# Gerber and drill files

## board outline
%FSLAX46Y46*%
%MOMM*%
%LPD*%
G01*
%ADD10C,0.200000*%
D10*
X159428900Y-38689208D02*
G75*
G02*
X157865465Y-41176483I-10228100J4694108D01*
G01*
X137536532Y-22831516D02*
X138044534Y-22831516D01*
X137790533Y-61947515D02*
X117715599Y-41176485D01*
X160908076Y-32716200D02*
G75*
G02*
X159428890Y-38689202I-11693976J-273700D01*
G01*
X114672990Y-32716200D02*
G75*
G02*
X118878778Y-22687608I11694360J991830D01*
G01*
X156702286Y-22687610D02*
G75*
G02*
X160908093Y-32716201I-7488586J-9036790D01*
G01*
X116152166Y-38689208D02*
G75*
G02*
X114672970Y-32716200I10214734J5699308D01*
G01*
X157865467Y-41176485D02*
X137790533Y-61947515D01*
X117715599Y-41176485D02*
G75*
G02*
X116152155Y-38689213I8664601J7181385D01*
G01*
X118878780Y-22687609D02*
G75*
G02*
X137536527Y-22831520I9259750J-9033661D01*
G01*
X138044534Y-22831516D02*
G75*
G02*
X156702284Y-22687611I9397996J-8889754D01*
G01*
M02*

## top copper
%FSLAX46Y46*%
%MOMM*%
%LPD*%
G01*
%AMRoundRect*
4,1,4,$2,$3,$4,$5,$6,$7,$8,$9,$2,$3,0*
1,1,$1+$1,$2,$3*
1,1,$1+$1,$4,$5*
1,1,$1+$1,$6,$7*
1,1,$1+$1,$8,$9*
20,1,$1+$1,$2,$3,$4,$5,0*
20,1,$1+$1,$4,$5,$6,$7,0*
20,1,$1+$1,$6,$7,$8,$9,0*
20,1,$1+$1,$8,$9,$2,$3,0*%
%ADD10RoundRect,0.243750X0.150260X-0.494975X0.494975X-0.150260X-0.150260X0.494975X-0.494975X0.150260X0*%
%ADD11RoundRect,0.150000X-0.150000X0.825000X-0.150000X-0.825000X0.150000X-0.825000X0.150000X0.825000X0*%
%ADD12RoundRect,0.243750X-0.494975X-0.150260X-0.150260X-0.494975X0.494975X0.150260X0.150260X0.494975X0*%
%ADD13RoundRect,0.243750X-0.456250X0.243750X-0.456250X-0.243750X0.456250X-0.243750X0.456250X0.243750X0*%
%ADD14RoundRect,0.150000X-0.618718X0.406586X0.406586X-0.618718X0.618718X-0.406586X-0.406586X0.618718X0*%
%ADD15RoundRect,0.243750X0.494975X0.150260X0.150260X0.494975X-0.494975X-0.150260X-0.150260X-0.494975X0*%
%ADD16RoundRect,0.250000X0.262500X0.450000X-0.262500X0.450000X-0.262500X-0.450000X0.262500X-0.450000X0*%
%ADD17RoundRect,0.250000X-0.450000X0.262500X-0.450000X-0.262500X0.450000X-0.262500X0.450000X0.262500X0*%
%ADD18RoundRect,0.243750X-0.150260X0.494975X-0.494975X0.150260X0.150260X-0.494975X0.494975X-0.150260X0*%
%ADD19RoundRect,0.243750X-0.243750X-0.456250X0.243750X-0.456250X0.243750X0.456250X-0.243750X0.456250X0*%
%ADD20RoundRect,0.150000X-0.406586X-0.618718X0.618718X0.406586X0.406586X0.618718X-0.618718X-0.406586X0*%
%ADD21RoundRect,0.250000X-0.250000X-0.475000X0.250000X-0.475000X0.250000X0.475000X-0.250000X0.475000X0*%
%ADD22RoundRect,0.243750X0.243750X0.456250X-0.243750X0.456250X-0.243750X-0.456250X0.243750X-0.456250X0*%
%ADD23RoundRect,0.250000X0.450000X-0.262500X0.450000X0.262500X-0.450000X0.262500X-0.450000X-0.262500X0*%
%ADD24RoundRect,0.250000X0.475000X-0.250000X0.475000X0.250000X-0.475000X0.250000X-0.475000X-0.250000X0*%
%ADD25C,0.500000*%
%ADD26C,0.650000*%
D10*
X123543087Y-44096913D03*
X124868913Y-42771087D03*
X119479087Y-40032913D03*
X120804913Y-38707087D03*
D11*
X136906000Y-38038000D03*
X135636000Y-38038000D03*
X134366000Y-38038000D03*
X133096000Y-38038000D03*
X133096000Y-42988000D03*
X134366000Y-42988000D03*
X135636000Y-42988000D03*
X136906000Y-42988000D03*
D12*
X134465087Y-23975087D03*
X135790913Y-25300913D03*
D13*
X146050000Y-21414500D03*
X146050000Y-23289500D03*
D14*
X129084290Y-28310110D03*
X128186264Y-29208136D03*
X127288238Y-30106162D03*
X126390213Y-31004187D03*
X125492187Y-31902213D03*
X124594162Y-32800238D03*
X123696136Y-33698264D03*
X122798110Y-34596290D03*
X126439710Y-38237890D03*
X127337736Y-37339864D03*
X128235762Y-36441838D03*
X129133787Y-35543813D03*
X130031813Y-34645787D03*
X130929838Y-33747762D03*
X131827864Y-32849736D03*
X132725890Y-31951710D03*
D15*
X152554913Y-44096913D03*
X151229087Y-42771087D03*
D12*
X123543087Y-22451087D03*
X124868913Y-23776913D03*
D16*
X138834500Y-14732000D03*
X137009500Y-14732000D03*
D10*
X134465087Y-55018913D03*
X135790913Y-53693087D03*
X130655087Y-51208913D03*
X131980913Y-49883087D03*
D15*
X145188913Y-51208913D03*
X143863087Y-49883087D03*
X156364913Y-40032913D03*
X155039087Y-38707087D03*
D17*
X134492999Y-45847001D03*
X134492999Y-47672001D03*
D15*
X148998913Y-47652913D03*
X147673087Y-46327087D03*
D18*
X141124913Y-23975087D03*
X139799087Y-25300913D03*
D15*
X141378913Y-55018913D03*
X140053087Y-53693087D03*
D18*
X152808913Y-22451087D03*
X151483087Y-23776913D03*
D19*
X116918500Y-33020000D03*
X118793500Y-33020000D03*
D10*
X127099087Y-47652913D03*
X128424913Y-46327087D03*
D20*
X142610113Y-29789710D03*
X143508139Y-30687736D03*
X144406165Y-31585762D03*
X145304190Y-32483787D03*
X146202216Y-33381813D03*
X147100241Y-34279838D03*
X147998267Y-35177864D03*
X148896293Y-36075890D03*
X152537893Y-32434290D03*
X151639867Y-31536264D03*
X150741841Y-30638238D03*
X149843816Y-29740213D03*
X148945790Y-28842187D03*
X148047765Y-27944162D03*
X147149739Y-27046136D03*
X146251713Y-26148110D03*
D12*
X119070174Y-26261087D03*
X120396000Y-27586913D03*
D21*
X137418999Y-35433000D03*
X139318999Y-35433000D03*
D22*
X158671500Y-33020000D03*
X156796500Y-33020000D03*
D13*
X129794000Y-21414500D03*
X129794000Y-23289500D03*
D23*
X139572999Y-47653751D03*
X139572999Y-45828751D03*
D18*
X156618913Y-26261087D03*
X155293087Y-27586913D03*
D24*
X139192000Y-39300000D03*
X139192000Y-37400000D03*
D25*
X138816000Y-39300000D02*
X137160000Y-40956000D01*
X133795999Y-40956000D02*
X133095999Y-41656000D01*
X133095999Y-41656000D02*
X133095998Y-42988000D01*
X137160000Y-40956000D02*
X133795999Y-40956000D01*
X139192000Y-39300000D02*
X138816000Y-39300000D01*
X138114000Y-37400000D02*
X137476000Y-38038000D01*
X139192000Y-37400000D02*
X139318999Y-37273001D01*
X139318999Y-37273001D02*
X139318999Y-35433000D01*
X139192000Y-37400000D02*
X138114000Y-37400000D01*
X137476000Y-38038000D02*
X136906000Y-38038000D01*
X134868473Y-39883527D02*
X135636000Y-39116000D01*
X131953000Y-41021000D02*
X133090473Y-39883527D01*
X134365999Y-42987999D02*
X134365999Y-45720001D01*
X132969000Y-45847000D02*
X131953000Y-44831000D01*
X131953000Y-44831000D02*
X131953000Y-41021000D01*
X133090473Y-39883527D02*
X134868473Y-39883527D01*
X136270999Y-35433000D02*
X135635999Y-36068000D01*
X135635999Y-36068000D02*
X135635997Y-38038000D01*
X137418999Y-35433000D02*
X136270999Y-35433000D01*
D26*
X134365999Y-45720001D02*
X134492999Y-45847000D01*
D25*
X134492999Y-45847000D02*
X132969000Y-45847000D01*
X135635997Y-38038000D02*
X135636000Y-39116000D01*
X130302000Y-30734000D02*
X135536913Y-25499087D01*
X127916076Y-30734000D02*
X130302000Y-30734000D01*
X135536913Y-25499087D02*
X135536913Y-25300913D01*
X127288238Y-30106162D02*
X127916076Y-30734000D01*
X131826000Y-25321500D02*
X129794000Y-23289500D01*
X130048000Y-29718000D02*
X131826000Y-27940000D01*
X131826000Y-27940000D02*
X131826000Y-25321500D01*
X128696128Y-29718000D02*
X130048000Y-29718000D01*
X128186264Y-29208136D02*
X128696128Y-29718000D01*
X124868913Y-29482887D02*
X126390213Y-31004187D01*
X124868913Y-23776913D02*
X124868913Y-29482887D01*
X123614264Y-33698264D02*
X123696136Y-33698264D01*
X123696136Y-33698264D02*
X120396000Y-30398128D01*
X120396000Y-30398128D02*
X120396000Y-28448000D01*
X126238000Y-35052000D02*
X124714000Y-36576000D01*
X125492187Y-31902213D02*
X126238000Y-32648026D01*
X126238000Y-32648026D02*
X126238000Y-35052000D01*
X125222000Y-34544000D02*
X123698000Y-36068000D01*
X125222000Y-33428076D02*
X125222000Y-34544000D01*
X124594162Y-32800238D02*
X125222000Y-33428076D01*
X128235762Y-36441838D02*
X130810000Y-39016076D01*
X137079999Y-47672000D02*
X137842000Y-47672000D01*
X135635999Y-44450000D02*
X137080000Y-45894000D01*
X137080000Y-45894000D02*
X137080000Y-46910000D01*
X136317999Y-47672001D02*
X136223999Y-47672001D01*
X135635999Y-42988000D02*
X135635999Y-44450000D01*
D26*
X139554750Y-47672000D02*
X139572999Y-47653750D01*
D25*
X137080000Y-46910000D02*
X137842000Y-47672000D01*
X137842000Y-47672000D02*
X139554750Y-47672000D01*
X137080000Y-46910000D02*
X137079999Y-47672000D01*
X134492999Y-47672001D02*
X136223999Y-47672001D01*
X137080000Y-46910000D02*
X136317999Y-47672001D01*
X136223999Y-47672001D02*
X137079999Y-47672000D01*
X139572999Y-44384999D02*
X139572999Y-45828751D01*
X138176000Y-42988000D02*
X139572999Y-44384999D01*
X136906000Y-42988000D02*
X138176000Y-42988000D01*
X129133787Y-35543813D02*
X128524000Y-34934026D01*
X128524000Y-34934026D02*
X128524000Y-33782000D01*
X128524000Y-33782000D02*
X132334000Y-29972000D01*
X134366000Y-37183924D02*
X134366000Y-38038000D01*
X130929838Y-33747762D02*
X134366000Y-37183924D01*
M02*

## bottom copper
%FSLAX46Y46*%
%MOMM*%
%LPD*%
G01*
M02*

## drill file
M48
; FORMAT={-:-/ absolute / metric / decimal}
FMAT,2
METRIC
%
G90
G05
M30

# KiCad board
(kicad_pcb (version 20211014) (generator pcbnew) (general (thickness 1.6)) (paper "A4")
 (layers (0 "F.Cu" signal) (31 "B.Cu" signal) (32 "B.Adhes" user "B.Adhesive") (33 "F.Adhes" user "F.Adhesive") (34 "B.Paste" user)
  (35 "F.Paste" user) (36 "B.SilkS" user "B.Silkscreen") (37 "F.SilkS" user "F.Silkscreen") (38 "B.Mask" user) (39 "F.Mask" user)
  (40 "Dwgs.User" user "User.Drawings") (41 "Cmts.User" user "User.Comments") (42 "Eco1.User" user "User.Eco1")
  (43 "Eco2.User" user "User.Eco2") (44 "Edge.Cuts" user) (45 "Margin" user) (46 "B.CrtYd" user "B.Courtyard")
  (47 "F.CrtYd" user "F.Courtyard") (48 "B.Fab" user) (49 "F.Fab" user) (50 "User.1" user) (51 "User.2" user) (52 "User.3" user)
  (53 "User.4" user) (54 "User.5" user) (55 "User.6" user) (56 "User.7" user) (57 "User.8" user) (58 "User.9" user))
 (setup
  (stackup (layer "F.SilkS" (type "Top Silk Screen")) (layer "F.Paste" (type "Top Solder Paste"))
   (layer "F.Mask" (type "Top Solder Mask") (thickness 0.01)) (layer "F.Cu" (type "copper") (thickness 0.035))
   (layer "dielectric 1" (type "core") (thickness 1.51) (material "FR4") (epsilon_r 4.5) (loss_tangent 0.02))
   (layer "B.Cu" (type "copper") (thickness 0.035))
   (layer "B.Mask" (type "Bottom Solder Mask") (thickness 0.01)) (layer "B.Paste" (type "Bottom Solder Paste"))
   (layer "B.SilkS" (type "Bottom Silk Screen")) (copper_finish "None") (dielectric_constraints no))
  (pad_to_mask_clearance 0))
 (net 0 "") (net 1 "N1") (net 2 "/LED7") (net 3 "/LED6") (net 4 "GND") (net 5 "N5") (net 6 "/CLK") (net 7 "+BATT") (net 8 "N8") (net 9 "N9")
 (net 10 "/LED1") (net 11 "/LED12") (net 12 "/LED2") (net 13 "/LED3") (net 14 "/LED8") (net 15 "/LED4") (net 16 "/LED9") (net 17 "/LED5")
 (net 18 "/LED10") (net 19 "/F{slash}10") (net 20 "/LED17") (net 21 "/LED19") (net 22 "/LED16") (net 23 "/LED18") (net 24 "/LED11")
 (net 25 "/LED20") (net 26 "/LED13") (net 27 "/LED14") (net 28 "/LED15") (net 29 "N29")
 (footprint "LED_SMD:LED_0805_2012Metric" (layer "F.Cu") (at 124.206 43.434 45)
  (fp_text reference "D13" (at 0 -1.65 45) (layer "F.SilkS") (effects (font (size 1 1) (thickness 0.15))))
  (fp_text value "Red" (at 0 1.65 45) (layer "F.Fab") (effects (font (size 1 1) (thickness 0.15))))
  (pad "1" smd roundrect (at -0.9375 0 45) (size 0.975 1.4) (layers "F.Cu" "F.Paste" "F.Mask") (roundrect_rratio 0.25) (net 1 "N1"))
  (pad "2" smd roundrect (at 0.9375 0 45) (size 0.975 1.4) (layers "F.Cu" "F.Paste" "F.Mask") (roundrect_rratio 0.25) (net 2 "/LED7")))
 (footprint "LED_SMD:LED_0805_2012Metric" (layer "F.Cu") (at 120.142 39.37 45)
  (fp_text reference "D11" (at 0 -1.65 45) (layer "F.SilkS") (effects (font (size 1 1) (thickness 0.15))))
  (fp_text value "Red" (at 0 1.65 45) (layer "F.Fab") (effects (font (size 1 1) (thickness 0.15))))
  (pad "1" smd roundrect (at -0.9375 0 45) (size 0.975 1.4) (layers "F.Cu" "F.Paste" "F.Mask") (roundrect_rratio 0.25) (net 1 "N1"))
  (pad "2" smd roundrect (at 0.9375 0 45) (size 0.975 1.4) (layers "F.Cu" "F.Paste" "F.Mask") (roundrect_rratio 0.25) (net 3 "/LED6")))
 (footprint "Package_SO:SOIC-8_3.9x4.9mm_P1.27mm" (layer "F.Cu") (at 135.001 40.513 -90)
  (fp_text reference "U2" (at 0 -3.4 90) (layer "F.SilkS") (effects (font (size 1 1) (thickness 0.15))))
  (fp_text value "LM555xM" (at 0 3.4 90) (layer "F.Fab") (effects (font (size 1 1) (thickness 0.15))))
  (pad "1" smd roundrect (at -2.475 -1.905 270) (size 1.95 0.6) (layers "F.Cu" "F.Paste" "F.Mask") (roundrect_rratio 0.25) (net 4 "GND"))
  (pad "2" smd roundrect (at -2.475 -0.635 270) (size 1.95 0.6) (layers "F.Cu" "F.Paste" "F.Mask") (roundrect_rratio 0.25) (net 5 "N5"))
  (pad "3" smd roundrect (at -2.475 0.635 270) (size 1.95 0.6) (layers "F.Cu" "F.Paste" "F.Mask") (roundrect_rratio 0.25) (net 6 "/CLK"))
  (pad "4" smd roundrect (at -2.475 1.905 270) (size 1.95 0.6) (layers "F.Cu" "F.Paste" "F.Mask") (roundrect_rratio 0.25) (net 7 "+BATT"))
  (pad "5" smd roundrect (at 2.475 1.905 270) (size 1.95 0.6) (layers "F.Cu" "F.Paste" "F.Mask") (roundrect_rratio 0.25) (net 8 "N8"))
  (pad "6" smd roundrect (at 2.475 0.635 270) (size 1.95 0.6) (layers "F.Cu" "F.Paste" "F.Mask") (roundrect_rratio 0.25) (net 5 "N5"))
  (pad "7" smd roundrect (at 2.475 -0.635 270) (size 1.95 0.6) (layers "F.Cu" "F.Paste" "F.Mask") (roundrect_rratio 0.25) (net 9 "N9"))
  (pad "8" smd roundrect (at 2.475 -1.905 270) (size 1.95 0.6) (layers "F.Cu" "F.Paste" "F.Mask") (roundrect_rratio 0.25) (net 7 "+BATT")))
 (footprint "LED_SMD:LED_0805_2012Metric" (layer "F.Cu") (at 135.128 24.638 -45)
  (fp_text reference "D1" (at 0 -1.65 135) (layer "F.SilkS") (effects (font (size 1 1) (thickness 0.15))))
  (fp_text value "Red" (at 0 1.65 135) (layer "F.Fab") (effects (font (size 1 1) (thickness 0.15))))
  (pad "1" smd roundrect (at -0.9375 0 315) (size 0.975 1.4) (layers "F.Cu" "F.Paste" "F.Mask") (roundrect_rratio 0.25) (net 1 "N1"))
  (pad "2" smd roundrect (at 0.9375 0 315) (size 0.975 1.4) (layers "F.Cu" "F.Paste" "F.Mask") (roundrect_rratio 0.25) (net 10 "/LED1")))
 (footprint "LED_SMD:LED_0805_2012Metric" (layer "F.Cu") (at 146.05 22.352 -90)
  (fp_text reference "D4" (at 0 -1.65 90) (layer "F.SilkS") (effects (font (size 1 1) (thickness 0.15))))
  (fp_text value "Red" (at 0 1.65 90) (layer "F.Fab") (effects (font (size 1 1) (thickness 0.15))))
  (pad "1" smd roundrect (at -0.9375 0 270) (size 0.975 1.4) (layers "F.Cu" "F.Paste" "F.Mask") (roundrect_rratio 0.25) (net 1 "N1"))
  (pad "2" smd roundrect (at 0.9375 0 270) (size 0.975 1.4) (layers "F.Cu" "F.Paste" "F.Mask") (roundrect_rratio 0.25) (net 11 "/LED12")))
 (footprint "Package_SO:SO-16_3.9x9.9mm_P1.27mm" (layer "F.Cu") (at 127.762 33.274 -45)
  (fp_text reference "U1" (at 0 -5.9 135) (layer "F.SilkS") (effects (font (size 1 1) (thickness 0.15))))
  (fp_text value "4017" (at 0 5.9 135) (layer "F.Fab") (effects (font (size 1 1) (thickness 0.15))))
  (pad "1" smd roundrect (at -2.575 -4.445 315) (size 1.75 0.6) (layers "F.Cu" "F.Paste" "F.Mask") (roundrect_rratio 0.25) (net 3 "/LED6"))
  (pad "2" smd roundrect (at -2.575 -3.175 315) (size 1.75 0.6) (layers "F.Cu" "F.Paste" "F.Mask") (roundrect_rratio 0.25) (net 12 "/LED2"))
  (pad "3" smd roundrect (at -2.575 -1.905 315) (size 1.75 0.6) (layers "F.Cu" "F.Paste" "F.Mask") (roundrect_rratio 0.25) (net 10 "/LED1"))
  (pad "4" smd roundrect (at -2.575 -0.635 315) (size 1.75 0.6) (layers "F.Cu" "F.Paste" "F.Mask") (roundrect_rratio 0.25) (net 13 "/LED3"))
  (pad "5" smd roundrect (at -2.575 0.635 315) (size 1.75 0.6) (layers "F.Cu" "F.Paste" "F.Mask") (roundrect_rratio 0.25) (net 2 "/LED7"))
  (pad "6" smd roundrect (at -2.575 1.905 315) (size 1.75 0.6) (layers "F.Cu" "F.Paste" "F.Mask") (roundrect_rratio 0.25) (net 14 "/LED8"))
  (pad "7" smd roundrect (at -2.575 3.175 315) (size 1.75 0.6) (layers "F.Cu" "F.Paste" "F.Mask") (roundrect_rratio 0.25) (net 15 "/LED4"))
  (pad "8" smd roundrect (at -2.575 4.445 315) (size 1.75 0.6) (layers "F.Cu" "F.Paste" "F.Mask") (roundrect_rratio 0.25) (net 4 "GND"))
  (pad "9" smd roundrect (at 2.575 4.445 315) (size 1.75 0.6) (layers "F.Cu" "F.Paste" "F.Mask") (roundrect_rratio 0.25) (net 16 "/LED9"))
  (pad "10" smd roundrect (at 2.575 3.175 315) (size 1.75 0.6) (layers "F.Cu" "F.Paste" "F.Mask") (roundrect_rratio 0.25) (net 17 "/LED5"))
  (pad "11" smd roundrect (at 2.575 1.905 315) (size 1.75 0.6) (layers "F.Cu" "F.Paste" "F.Mask") (roundrect_rratio 0.25) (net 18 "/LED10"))
  (pad "12" smd roundrect (at 2.575 0.635 315) (size 1.75 0.6) (layers "F.Cu" "F.Paste" "F.Mask") (roundrect_rratio 0.25)
   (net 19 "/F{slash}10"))
  (pad "13" smd roundrect (at 2.575 -0.635 315) (size 1.75 0.6) (layers "F.Cu" "F.Paste" "F.Mask") (roundrect_rratio 0.25) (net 4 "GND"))
  (pad "14" smd roundrect (at 2.575 -1.905 315) (size 1.75 0.6) (layers "F.Cu" "F.Paste" "F.Mask") (roundrect_rratio 0.25) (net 6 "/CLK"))
  (pad "15" smd roundrect (at 2.575 -3.175 315) (size 1.75 0.6) (layers "F.Cu" "F.Paste" "F.Mask") (roundrect_rratio 0.25) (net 4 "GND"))
  (pad "16" smd roundrect (at 2.575 -4.445 315) (size 1.75 0.6) (layers "F.Cu" "F.Paste" "F.Mask") (roundrect_rratio 0.25) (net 7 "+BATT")))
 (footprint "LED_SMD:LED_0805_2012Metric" (layer "F.Cu") (at 151.892 43.434 135)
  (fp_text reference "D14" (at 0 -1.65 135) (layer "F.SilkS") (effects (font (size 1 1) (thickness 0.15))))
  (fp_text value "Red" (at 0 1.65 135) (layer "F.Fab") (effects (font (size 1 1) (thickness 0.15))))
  (pad "1" smd roundrect (at -0.9375 0 135) (size 0.975 1.4) (layers "F.Cu" "F.Paste" "F.Mask") (roundrect_rratio 0.25) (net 1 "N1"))
  (pad "2" smd roundrect (at 0.9375 0 135) (size 0.975 1.4) (layers "F.Cu" "F.Paste" "F.Mask") (roundrect_rratio 0.25) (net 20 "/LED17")))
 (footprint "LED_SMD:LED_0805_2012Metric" (layer "F.Cu") (at 124.206 23.114 -45)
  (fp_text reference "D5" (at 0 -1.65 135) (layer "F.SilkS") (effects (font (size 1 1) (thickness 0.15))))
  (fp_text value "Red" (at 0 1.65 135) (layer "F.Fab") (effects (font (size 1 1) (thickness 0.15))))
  (pad "1" smd roundrect (at -0.9375 0 315) (size 0.975 1.4) (layers "F.Cu" "F.Paste" "F.Mask") (roundrect_rratio 0.25) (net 1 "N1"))
  (pad "2" smd roundrect (at 0.9375 0 315) (size 0.975 1.4) (layers "F.Cu" "F.Paste" "F.Mask") (roundrect_rratio 0.25) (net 13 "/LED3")))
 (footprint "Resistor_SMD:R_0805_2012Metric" (layer "F.Cu") (at 137.922 14.732 180)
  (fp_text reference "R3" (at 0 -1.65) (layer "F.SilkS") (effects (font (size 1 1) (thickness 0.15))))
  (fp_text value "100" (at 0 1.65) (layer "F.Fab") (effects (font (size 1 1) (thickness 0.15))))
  (pad "1" smd roundrect (at -0.9125 0 180) (size 1.025 1.4) (layers "F.Cu" "F.Paste" "F.Mask") (roundrect_rratio 0.243902) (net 4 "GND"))
  (pad "2" smd roundrect (at 0.9125 0 180) (size 1.025 1.4) (layers "F.Cu" "F.Paste" "F.Mask") (roundrect_rratio 0.243902) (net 1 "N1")))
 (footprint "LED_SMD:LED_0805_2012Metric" (layer "F.Cu") (at 135.128 54.356 45)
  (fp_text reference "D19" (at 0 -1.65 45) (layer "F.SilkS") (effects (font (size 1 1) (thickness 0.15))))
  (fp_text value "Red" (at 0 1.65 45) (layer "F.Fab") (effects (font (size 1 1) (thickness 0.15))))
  (pad "1" smd roundrect (at -0.9375 0 45) (size 0.975 1.4) (layers "F.Cu" "F.Paste" "F.Mask") (roundrect_rratio 0.25) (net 1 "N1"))
  (pad "2" smd roundrect (at 0.9375 0 45) (size 0.975 1.4) (layers "F.Cu" "F.Paste" "F.Mask") (roundrect_rratio 0.25) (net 18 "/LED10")))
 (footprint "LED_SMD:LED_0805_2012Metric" (layer "F.Cu") (at 131.318 50.546 45)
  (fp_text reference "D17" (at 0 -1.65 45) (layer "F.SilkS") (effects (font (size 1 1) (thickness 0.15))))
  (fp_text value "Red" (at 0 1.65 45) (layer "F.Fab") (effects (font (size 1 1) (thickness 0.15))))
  (pad "1" smd roundrect (at -0.9375 0 45) (size 0.975 1.4) (layers "F.Cu" "F.Paste" "F.Mask") (roundrect_rratio 0.25) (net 1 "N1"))
  (pad "2" smd roundrect (at 0.9375 0 45) (size 0.975 1.4) (layers "F.Cu" "F.Paste" "F.Mask") (roundrect_rratio 0.25) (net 16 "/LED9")))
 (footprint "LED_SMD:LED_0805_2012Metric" (layer "F.Cu") (at 144.526 50.546 135)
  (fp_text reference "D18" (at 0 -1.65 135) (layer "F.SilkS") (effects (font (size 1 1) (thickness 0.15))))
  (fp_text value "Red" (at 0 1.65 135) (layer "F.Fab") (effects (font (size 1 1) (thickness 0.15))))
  (pad "1" smd roundrect (at -0.9375 0 135) (size 0.975 1.4) (layers "F.Cu" "F.Paste" "F.Mask") (roundrect_rratio 0.25) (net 1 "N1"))
  (pad "2" smd roundrect (at 0.9375 0 135) (size 0.975 1.4) (layers "F.Cu" "F.Paste" "F.Mask") (roundrect_rratio 0.25) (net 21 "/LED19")))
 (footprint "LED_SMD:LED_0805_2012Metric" (layer "F.Cu") (at 155.702 39.37 135)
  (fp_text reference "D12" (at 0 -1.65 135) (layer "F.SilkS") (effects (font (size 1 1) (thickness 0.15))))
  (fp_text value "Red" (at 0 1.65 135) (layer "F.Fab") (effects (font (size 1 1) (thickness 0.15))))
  (pad "1" smd roundrect (at -0.9375 0 135) (size 0.975 1.4) (layers "F.Cu" "F.Paste" "F.Mask") (roundrect_rratio 0.25) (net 1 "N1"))
  (pad "2" smd roundrect (at 0.9375 0 135) (size 0.975 1.4) (layers "F.Cu" "F.Paste" "F.Mask") (roundrect_rratio 0.25) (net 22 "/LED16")))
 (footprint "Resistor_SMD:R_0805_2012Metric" (layer "F.Cu") (at 134.492999 46.759501 -90)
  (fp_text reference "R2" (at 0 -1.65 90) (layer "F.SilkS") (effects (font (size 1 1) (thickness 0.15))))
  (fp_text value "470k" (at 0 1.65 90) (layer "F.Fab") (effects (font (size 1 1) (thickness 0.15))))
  (pad "1" smd roundrect (at -0.9125 0 270) (size 1.025 1.4) (layers "F.Cu" "F.Paste" "F.Mask") (roundrect_rratio 0.243902) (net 5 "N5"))
  (pad "2" smd roundrect (at 0.9125 0 270) (size 1.025 1.4) (layers "F.Cu" "F.Paste" "F.Mask") (roundrect_rratio 0.243902) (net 9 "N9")))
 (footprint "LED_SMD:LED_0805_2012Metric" (layer "F.Cu") (at 148.336 46.99 135)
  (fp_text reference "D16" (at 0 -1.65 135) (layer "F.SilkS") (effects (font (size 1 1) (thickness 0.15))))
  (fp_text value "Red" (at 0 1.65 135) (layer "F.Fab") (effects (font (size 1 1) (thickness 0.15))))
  (pad "1" smd roundrect (at -0.9375 0 135) (size 0.975 1.4) (layers "F.Cu" "F.Paste" "F.Mask") (roundrect_rratio 0.25) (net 1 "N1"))
  (pad "2" smd roundrect (at 0.9375 0 135) (size 0.975 1.4) (layers "F.Cu" "F.Paste" "F.Mask") (roundrect_rratio 0.25) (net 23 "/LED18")))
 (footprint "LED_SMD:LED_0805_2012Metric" (layer "F.Cu") (at 140.462 24.638 -135)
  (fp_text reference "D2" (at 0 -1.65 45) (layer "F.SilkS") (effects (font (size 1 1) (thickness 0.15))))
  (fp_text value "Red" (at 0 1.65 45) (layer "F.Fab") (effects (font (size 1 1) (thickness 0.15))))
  (pad "1" smd roundrect (at -0.9375 0 225) (size 0.975 1.4) (layers "F.Cu" "F.Paste" "F.Mask") (roundrect_rratio 0.25) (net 1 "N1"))
  (pad "2" smd roundrect (at 0.9375 0 225) (size 0.975 1.4) (layers "F.Cu" "F.Paste" "F.Mask") (roundrect_rratio 0.25) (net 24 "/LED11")))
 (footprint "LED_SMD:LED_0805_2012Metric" (layer "F.Cu") (at 140.716 54.356 135)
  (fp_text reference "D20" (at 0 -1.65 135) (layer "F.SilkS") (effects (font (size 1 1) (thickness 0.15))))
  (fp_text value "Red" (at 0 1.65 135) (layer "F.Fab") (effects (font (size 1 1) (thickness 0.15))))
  (pad "1" smd roundrect (at -0.9375 0 135) (size 0.975 1.4) (layers "F.Cu" "F.Paste" "F.Mask") (roundrect_rratio 0.25) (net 1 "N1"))
  (pad "2" smd roundrect (at 0.9375 0 135) (size 0.975 1.4) (layers "F.Cu" "F.Paste" "F.Mask") (roundrect_rratio 0.25) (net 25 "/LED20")))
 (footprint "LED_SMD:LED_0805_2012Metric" (layer "F.Cu") (at 152.146 23.114 -135)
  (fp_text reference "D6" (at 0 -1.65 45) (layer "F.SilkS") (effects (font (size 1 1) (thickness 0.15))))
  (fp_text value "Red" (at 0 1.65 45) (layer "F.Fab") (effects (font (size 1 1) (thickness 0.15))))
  (pad "1" smd roundrect (at -0.9375 0 225) (size 0.975 1.4) (layers "F.Cu" "F.Paste" "F.Mask") (roundrect_rratio 0.25) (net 1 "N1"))
  (pad "2" smd roundrect (at 0.9375 0 225) (size 0.975 1.4) (layers "F.Cu" "F.Paste" "F.Mask") (roundrect_rratio 0.25) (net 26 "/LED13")))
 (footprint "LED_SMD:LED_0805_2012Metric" (layer "F.Cu") (at 117.856 33.02)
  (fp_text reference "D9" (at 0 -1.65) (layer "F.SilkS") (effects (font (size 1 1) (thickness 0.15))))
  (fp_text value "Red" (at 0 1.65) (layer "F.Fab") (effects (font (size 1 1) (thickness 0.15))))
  (pad "1" smd roundrect (at -0.9375 0) (size 0.975 1.4) (layers "F.Cu" "F.Paste" "F.Mask") (roundrect_rratio 0.25) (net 1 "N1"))
  (pad "2" smd roundrect (at 0.9375 0) (size 0.975 1.4) (layers "F.Cu" "F.Paste" "F.Mask") (roundrect_rratio 0.25) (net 17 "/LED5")))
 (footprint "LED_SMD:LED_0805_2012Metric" (layer "F.Cu") (at 127.762 46.99 45)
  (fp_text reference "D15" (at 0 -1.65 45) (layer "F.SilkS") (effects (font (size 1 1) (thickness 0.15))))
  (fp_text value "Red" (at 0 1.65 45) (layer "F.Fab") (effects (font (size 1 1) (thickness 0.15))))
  (pad "1" smd roundrect (at -0.9375 0 45) (size 0.975 1.4) (layers "F.Cu" "F.Paste" "F.Mask") (roundrect_rratio 0.25) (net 1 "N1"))
  (pad "2" smd roundrect (at 0.9375 0 45) (size 0.975 1.4) (layers "F.Cu" "F.Paste" "F.Mask") (roundrect_rratio 0.25) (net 14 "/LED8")))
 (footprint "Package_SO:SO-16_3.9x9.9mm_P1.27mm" (layer "F.Cu") (at 147.574003 31.112 45)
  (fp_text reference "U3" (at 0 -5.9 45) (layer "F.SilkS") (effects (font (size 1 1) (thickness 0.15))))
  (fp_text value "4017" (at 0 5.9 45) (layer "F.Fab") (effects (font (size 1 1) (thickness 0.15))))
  (pad "1" smd roundrect (at -2.575 -4.445 45) (size 1.75 0.6) (layers "F.Cu" "F.Paste" "F.Mask") (roundrect_rratio 0.25) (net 22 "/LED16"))
  (pad "2" smd roundrect (at -2.575 -3.175 45) (size 1.75 0.6) (layers "F.Cu" "F.Paste" "F.Mask") (roundrect_rratio 0.25) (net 11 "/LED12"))
  (pad "3" smd roundrect (at -2.575 -1.905 45) (size 1.75 0.6) (layers "F.Cu" "F.Paste" "F.Mask") (roundrect_rratio 0.25) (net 24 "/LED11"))
  (pad "4" smd roundrect (at -2.575 -0.635 45) (size 1.75 0.6) (layers "F.Cu" "F.Paste" "F.Mask") (roundrect_rratio 0.25) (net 26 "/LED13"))
  (pad "5" smd roundrect (at -2.575 0.635 45) (size 1.75 0.6) (layers "F.Cu" "F.Paste" "F.Mask") (roundrect_rratio 0.25) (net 20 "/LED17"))
  (pad "6" smd roundrect (at -2.575 1.905 45) (size 1.75 0.6) (layers "F.Cu" "F.Paste" "F.Mask") (roundrect_rratio 0.25) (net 23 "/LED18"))
  (pad "7" smd roundrect (at -2.575 3.175 45) (size 1.75 0.6) (layers "F.Cu" "F.Paste" "F.Mask") (roundrect_rratio 0.25) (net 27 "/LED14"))
  (pad "8" smd roundrect (at -2.575 4.445 45) (size 1.75 0.6) (layers "F.Cu" "F.Paste" "F.Mask") (roundrect_rratio 0.25) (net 4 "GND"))
  (pad "9" smd roundrect (at 2.575 4.445 45) (size 1.75 0.6) (layers "F.Cu" "F.Paste" "F.Mask") (roundrect_rratio 0.25) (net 21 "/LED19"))
  (pad "10" smd roundrect (at 2.575 3.175 45) (size 1.75 0.6) (layers "F.Cu" "F.Paste" "F.Mask") (roundrect_rratio 0.25) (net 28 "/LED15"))
  (pad "11" smd roundrect (at 2.575 1.905 45) (size 1.75 0.6) (layers "F.Cu" "F.Paste" "F.Mask") (roundrect_rratio 0.25) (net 25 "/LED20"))
  (pad "12" smd roundrect (at 2.575 0.635 45) (size 1.75 0.6) (layers "F.Cu" "F.Paste" "F.Mask") (roundrect_rratio 0.25) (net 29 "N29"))
  (pad "13" smd roundrect (at 2.575 -0.635 45) (size 1.75 0.6) (layers "F.Cu" "F.Paste" "F.Mask") (roundrect_rratio 0.25) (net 4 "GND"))
  (pad "14" smd roundrect (at 2.575 -1.905 45) (size 1.75 0.6) (layers "F.Cu" "F.Paste" "F.Mask") (roundrect_rratio 0.25)
   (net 19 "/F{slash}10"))
  (pad "15" smd roundrect (at 2.575 -3.175 45) (size 1.75 0.6) (layers "F.Cu" "F.Paste" "F.Mask") (roundrect_rratio 0.25) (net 4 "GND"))
  (pad "16" smd roundrect (at 2.575 -4.445 45) (size 1.75 0.6) (layers "F.Cu" "F.Paste" "F.Mask") (roundrect_rratio 0.25) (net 7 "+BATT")))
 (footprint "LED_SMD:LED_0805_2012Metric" (layer "F.Cu") (at 119.733087 26.924 -45)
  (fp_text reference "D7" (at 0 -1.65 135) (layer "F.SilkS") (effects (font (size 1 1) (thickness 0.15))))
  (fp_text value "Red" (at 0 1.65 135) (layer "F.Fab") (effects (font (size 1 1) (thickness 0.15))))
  (pad "1" smd roundrect (at -0.9375 0 315) (size 0.975 1.4) (layers "F.Cu" "F.Paste" "F.Mask") (roundrect_rratio 0.25) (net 1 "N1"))
  (pad "2" smd roundrect (at 0.9375 0 315) (size 0.975 1.4) (layers "F.Cu" "F.Paste" "F.Mask") (roundrect_rratio 0.25) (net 15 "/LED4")))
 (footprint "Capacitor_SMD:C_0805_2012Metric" (layer "F.Cu") (at 138.368999 35.433)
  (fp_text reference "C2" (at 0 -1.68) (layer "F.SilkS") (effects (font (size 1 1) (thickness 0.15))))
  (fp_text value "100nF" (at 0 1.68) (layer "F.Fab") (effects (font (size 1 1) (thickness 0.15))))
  (pad "1" smd roundrect (at -0.95 0) (size 1 1.45) (layers "F.Cu" "F.Paste" "F.Mask") (roundrect_rratio 0.25) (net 5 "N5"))
  (pad "2" smd roundrect (at 0.95 0) (size 1 1.45) (layers "F.Cu" "F.Paste" "F.Mask") (roundrect_rratio 0.25) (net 4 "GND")))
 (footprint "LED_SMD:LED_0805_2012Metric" (layer "F.Cu") (at 157.734 33.02 180)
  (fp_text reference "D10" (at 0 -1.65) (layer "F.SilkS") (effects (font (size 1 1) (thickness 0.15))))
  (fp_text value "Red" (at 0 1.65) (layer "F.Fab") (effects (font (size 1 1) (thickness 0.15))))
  (pad "1" smd roundrect (at -0.9375 0 180) (size 0.975 1.4) (layers "F.Cu" "F.Paste" "F.Mask") (roundrect_rratio 0.25) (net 1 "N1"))
  (pad "2" smd roundrect (at 0.9375 0 180) (size 0.975 1.4) (layers "F.Cu" "F.Paste" "F.Mask") (roundrect_rratio 0.25) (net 28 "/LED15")))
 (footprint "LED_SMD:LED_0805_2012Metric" (layer "F.Cu") (at 129.794 22.352 -90)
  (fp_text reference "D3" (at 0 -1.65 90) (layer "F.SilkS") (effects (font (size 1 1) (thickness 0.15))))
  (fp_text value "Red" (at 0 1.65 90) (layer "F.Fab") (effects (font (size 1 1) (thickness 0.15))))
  (pad "1" smd roundrect (at -0.9375 0 270) (size 0.975 1.4) (layers "F.Cu" "F.Paste" "F.Mask") (roundrect_rratio 0.25) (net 1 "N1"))
  (pad "2" smd roundrect (at 0.9375 0 270) (size 0.975 1.4) (layers "F.Cu" "F.Paste" "F.Mask") (roundrect_rratio 0.25) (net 12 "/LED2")))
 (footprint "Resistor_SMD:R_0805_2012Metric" (layer "F.Cu") (at 139.572999 46.741251 90)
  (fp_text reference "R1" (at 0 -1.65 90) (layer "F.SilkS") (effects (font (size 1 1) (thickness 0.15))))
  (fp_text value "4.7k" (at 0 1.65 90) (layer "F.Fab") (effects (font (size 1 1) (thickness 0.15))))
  (pad "1" smd roundrect (at -0.9125 0 90) (size 1.025 1.4) (layers "F.Cu" "F.Paste" "F.Mask") (roundrect_rratio 0.243902) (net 9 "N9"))
  (pad "2" smd roundrect (at 0.9125 0 90) (size 1.025 1.4) (layers "F.Cu" "F.Paste" "F.Mask") (roundrect_rratio 0.243902) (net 7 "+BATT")))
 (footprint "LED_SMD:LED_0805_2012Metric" (layer "F.Cu") (at 155.956 26.924 -135)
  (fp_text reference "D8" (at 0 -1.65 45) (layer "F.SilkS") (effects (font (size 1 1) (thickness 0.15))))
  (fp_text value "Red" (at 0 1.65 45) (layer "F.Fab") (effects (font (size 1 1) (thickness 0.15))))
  (pad "1" smd roundrect (at -0.9375 0 225) (size 0.975 1.4) (layers "F.Cu" "F.Paste" "F.Mask") (roundrect_rratio 0.25) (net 1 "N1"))
  (pad "2" smd roundrect (at 0.9375 0 225) (size 0.975 1.4) (layers "F.Cu" "F.Paste" "F.Mask") (roundrect_rratio 0.25) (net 27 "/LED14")))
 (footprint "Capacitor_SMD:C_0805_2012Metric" (layer "F.Cu") (at 139.192 38.35 90)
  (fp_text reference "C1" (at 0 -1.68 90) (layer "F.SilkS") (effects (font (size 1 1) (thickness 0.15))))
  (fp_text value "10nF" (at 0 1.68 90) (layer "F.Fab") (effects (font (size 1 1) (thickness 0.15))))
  (pad "1" smd roundrect (at -0.95 0 90) (size 1 1.45) (layers "F.Cu" "F.Paste" "F.Mask") (roundrect_rratio 0.25) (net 8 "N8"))
  (pad "2" smd roundrect (at 0.95 0 90) (size 1 1.45) (layers "F.Cu" "F.Paste" "F.Mask") (roundrect_rratio 0.25) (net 4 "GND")))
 (gr_arc (start 159.4289 38.689208) (mid 158.728696 39.984083) (end 157.865467 41.176485) (layer "Edge.Cuts") (width 0.2))
 (gr_line (start 137.536532 22.831516) (end 138.044534 22.831516) (layer "Edge.Cuts") (width 0.2))
 (gr_line (start 137.790533 61.947515) (end 117.715599 41.176485) (layer "Edge.Cuts") (width 0.2))
 (gr_arc (start 160.908076 32.7162) (mid 160.568299 35.801715) (end 159.4289 38.689208) (layer "Edge.Cuts") (width 0.2))
 (gr_arc (start 114.67299 32.7162) (mid 115.544256 27.185384) (end 118.87878 22.68761) (layer "Edge.Cuts") (width 0.2))
 (gr_arc (start 156.702286 22.68761) (mid 160.03681 27.185384) (end 160.908076 32.7162) (layer "Edge.Cuts") (width 0.2))
 (gr_arc (start 116.152166 38.689208) (mid 115.012767 35.801715) (end 114.67299 32.7162) (layer "Edge.Cuts") (width 0.2))
 (gr_line (start 157.865467 41.176485) (end 137.790533 61.947515) (layer "Edge.Cuts") (width 0.2))
 (gr_arc (start 117.715599 41.176485) (mid 116.85237 39.984083) (end 116.152166 38.689208) (layer "Edge.Cuts") (width 0.2))
 (gr_arc (start 118.87878 22.687609) (mid 128.23831 18.78527) (end 137.536532 22.831516) (layer "Edge.Cuts") (width 0.2))
 (gr_arc (start 138.044534 22.831516) (mid 147.342756 18.78527) (end 156.702286 22.687609) (layer "Edge.Cuts") (width 0.2))
 (segment (start 138.816 39.3) (end 137.16 40.956) (width 0.5) (layer "F.Cu") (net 8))
 (segment (start 133.795999 40.956) (end 133.095999 41.656) (width 0.5) (layer "F.Cu") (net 8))
 (segment (start 133.095999 41.656) (end 133.095998 42.988) (width 0.5) (layer "F.Cu") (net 8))
 (segment (start 137.16 40.956) (end 133.795999 40.956) (width 0.5) (layer "F.Cu") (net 8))
 (segment (start 139.192 39.3) (end 138.816 39.3) (width 0.5) (layer "F.Cu") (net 8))
 (segment (start 138.114 37.4) (end 137.476 38.038) (width 0.5) (layer "F.Cu") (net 4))
 (segment (start 139.192 37.4) (end 139.318999 37.273001) (width 0.5) (layer "F.Cu") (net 4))
 (segment (start 139.318999 37.273001) (end 139.318999 35.433) (width 0.5) (layer "F.Cu") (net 4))
 (segment (start 139.192 37.4) (end 138.114 37.4) (width 0.5) (layer "F.Cu") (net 4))
 (segment (start 137.476 38.038) (end 136.906 38.038) (width 0.5) (layer "F.Cu") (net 4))
 (segment (start 134.868473 39.883527) (end 135.636 39.116) (width 0.5) (layer "F.Cu") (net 5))
 (segment (start 131.953 41.021) (end 133.090473 39.883527) (width 0.5) (layer "F.Cu") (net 5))
 (segment (start 134.365999 42.987999) (end 134.365999 45.720001) (width 0.5) (layer "F.Cu") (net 5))
 (segment (start 132.969 45.847) (end 131.953 44.831) (width 0.5) (layer "F.Cu") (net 5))
 (segment (start 131.953 44.831) (end 131.953 41.021) (width 0.5) (layer "F.Cu") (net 5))
 (segment (start 133.090473 39.883527) (end 134.868473 39.883527) (width 0.5) (layer "F.Cu") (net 5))
 (segment (start 136.270999 35.433) (end 135.635999 36.068) (width 0.5) (layer "F.Cu") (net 5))
 (segment (start 135.635999 36.068) (end 135.635997 38.038) (width 0.5) (layer "F.Cu") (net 5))
 (segment (start 137.418999 35.433) (end 136.270999 35.433) (width 0.5) (layer "F.Cu") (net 5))
 (segment (start 134.365999 45.720001) (end 134.492999 45.847) (width 0.65) (layer "F.Cu") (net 5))
 (segment (start 134.492999 45.847) (end 132.969 45.847) (width 0.5) (layer "F.Cu") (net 5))
 (segment (start 135.635997 38.038) (end 135.636 39.116) (width 0.5) (layer "F.Cu") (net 5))
 (segment (start 130.302 30.734) (end 135.536913 25.499087) (width 0.5) (layer "F.Cu") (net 10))
 (segment (start 127.916076 30.734) (end 130.302 30.734) (width 0.5) (layer "F.Cu") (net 10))
 (segment (start 135.536913 25.499087) (end 135.536913 25.300913) (width 0.5) (layer "F.Cu") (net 10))
 (segment (start 127.288238 30.106162) (end 127.916076 30.734) (width 0.5) (layer "F.Cu") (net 10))
 (segment (start 131.826 25.3215) (end 129.794 23.2895) (width 0.5) (layer "F.Cu") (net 12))
 (segment (start 130.048 29.718) (end 131.826 27.94) (width 0.5) (layer "F.Cu") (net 12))
 (segment (start 131.826 27.94) (end 131.826 25.3215) (width 0.5) (layer "F.Cu") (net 12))
 (segment (start 128.696128 29.718) (end 130.048 29.718) (width 0.5) (layer "F.Cu") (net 12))
 (segment (start 128.186264 29.208136) (end 128.696128 29.718) (width 0.5) (layer "F.Cu") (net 12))
 (segment (start 124.868913 29.482887) (end 126.390213 31.004187) (width 0.5) (layer "F.Cu") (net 13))
 (segment (start 124.868913 23.776913) (end 124.868913 29.482887) (width 0.5) (layer "F.Cu") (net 13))
 (segment (start 123.614264 33.698264) (end 123.696136 33.698264) (width 0.5) (layer "F.Cu") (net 15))
 (segment (start 123.696136 33.698264) (end 120.396 30.398128) (width 0.5) (layer "F.Cu") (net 15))
 (segment (start 120.396 30.398128) (end 120.396 28.448) (width 0.5) (layer "F.Cu") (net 15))
 (segment (start 126.238 35.052) (end 124.714 36.576) (width 0.5) (layer "F.Cu") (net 2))
 (segment (start 125.492187 31.902213) (end 126.238 32.648026) (width 0.5) (layer "F.Cu") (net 2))
 (segment (start 126.238 32.648026) (end 126.238 35.052) (width 0.5) (layer "F.Cu") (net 2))
 (segment (start 125.222 34.544) (end 123.698 36.068) (width 0.5) (layer "F.Cu") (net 14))
 (segment (start 125.222 33.428076) (end 125.222 34.544) (width 0.5) (layer "F.Cu") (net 14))
 (segment (start 124.594162 32.800238) (end 125.222 33.428076) (width 0.5) (layer "F.Cu") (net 14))
 (segment (start 128.235762 36.441838) (end 130.81 39.016076) (width 0.5) (layer "F.Cu") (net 18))
 (segment (start 137.079999 47.672) (end 137.842 47.672) (width 0.5) (layer "F.Cu") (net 9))
 (segment (start 135.635999 44.45) (end 137.08 45.894) (width 0.5) (layer "F.Cu") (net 9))
 (segment (start 137.08 45.894) (end 137.08 46.91) (width 0.5) (layer "F.Cu") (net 9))
 (segment (start 136.317999 47.672001) (end 136.223999 47.672001) (width 0.5) (layer "F.Cu") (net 9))
 (segment (start 135.635999 42.988) (end 135.635999 44.45) (width 0.5) (layer "F.Cu") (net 9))
 (segment (start 139.55475 47.672) (end 139.572999 47.65375) (width 0.65) (layer "F.Cu") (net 9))
 (segment (start 137.08 46.91) (end 137.842 47.672) (width 0.5) (layer "F.Cu") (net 9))
 (segment (start 137.842 47.672) (end 139.55475 47.672) (width 0.5) (layer "F.Cu") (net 9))
 (segment (start 137.08 46.91) (end 137.079999 47.672) (width 0.5) (layer "F.Cu") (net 9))
 (segment (start 134.492999 47.672001) (end 136.223999 47.672001) (width 0.5) (layer "F.Cu") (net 9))
 (segment (start 137.08 46.91) (end 136.317999 47.672001) (width 0.5) (layer "F.Cu") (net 9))
 (segment (start 136.223999 47.672001) (end 137.079999 47.672) (width 0.5) (layer "F.Cu") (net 9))
 (segment (start 139.572999 44.384999) (end 139.572999 45.828751) (width 0.5) (layer "F.Cu") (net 7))
 (segment (start 138.176 42.988) (end 139.572999 44.384999) (width 0.5) (layer "F.Cu") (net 7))
 (segment (start 136.906 42.988) (end 138.176 42.988) (width 0.5) (layer "F.Cu") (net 7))
 (segment (start 129.133787 35.543813) (end 128.524 34.934026) (width 0.5) (layer "F.Cu") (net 19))
 (segment (start 128.524 34.934026) (end 128.524 33.782) (width 0.5) (layer "F.Cu") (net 19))
 (segment (start 128.524 33.782) (end 132.334 29.972) (width 0.5) (layer "F.Cu") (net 19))
 (segment (start 134.366 37.183924) (end 134.366 38.038) (width 0.5) (layer "F.Cu") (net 6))
 (segment (start 130.929838 33.747762) (end 134.366 37.183924) (width 0.5) (layer "F.Cu") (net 6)))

